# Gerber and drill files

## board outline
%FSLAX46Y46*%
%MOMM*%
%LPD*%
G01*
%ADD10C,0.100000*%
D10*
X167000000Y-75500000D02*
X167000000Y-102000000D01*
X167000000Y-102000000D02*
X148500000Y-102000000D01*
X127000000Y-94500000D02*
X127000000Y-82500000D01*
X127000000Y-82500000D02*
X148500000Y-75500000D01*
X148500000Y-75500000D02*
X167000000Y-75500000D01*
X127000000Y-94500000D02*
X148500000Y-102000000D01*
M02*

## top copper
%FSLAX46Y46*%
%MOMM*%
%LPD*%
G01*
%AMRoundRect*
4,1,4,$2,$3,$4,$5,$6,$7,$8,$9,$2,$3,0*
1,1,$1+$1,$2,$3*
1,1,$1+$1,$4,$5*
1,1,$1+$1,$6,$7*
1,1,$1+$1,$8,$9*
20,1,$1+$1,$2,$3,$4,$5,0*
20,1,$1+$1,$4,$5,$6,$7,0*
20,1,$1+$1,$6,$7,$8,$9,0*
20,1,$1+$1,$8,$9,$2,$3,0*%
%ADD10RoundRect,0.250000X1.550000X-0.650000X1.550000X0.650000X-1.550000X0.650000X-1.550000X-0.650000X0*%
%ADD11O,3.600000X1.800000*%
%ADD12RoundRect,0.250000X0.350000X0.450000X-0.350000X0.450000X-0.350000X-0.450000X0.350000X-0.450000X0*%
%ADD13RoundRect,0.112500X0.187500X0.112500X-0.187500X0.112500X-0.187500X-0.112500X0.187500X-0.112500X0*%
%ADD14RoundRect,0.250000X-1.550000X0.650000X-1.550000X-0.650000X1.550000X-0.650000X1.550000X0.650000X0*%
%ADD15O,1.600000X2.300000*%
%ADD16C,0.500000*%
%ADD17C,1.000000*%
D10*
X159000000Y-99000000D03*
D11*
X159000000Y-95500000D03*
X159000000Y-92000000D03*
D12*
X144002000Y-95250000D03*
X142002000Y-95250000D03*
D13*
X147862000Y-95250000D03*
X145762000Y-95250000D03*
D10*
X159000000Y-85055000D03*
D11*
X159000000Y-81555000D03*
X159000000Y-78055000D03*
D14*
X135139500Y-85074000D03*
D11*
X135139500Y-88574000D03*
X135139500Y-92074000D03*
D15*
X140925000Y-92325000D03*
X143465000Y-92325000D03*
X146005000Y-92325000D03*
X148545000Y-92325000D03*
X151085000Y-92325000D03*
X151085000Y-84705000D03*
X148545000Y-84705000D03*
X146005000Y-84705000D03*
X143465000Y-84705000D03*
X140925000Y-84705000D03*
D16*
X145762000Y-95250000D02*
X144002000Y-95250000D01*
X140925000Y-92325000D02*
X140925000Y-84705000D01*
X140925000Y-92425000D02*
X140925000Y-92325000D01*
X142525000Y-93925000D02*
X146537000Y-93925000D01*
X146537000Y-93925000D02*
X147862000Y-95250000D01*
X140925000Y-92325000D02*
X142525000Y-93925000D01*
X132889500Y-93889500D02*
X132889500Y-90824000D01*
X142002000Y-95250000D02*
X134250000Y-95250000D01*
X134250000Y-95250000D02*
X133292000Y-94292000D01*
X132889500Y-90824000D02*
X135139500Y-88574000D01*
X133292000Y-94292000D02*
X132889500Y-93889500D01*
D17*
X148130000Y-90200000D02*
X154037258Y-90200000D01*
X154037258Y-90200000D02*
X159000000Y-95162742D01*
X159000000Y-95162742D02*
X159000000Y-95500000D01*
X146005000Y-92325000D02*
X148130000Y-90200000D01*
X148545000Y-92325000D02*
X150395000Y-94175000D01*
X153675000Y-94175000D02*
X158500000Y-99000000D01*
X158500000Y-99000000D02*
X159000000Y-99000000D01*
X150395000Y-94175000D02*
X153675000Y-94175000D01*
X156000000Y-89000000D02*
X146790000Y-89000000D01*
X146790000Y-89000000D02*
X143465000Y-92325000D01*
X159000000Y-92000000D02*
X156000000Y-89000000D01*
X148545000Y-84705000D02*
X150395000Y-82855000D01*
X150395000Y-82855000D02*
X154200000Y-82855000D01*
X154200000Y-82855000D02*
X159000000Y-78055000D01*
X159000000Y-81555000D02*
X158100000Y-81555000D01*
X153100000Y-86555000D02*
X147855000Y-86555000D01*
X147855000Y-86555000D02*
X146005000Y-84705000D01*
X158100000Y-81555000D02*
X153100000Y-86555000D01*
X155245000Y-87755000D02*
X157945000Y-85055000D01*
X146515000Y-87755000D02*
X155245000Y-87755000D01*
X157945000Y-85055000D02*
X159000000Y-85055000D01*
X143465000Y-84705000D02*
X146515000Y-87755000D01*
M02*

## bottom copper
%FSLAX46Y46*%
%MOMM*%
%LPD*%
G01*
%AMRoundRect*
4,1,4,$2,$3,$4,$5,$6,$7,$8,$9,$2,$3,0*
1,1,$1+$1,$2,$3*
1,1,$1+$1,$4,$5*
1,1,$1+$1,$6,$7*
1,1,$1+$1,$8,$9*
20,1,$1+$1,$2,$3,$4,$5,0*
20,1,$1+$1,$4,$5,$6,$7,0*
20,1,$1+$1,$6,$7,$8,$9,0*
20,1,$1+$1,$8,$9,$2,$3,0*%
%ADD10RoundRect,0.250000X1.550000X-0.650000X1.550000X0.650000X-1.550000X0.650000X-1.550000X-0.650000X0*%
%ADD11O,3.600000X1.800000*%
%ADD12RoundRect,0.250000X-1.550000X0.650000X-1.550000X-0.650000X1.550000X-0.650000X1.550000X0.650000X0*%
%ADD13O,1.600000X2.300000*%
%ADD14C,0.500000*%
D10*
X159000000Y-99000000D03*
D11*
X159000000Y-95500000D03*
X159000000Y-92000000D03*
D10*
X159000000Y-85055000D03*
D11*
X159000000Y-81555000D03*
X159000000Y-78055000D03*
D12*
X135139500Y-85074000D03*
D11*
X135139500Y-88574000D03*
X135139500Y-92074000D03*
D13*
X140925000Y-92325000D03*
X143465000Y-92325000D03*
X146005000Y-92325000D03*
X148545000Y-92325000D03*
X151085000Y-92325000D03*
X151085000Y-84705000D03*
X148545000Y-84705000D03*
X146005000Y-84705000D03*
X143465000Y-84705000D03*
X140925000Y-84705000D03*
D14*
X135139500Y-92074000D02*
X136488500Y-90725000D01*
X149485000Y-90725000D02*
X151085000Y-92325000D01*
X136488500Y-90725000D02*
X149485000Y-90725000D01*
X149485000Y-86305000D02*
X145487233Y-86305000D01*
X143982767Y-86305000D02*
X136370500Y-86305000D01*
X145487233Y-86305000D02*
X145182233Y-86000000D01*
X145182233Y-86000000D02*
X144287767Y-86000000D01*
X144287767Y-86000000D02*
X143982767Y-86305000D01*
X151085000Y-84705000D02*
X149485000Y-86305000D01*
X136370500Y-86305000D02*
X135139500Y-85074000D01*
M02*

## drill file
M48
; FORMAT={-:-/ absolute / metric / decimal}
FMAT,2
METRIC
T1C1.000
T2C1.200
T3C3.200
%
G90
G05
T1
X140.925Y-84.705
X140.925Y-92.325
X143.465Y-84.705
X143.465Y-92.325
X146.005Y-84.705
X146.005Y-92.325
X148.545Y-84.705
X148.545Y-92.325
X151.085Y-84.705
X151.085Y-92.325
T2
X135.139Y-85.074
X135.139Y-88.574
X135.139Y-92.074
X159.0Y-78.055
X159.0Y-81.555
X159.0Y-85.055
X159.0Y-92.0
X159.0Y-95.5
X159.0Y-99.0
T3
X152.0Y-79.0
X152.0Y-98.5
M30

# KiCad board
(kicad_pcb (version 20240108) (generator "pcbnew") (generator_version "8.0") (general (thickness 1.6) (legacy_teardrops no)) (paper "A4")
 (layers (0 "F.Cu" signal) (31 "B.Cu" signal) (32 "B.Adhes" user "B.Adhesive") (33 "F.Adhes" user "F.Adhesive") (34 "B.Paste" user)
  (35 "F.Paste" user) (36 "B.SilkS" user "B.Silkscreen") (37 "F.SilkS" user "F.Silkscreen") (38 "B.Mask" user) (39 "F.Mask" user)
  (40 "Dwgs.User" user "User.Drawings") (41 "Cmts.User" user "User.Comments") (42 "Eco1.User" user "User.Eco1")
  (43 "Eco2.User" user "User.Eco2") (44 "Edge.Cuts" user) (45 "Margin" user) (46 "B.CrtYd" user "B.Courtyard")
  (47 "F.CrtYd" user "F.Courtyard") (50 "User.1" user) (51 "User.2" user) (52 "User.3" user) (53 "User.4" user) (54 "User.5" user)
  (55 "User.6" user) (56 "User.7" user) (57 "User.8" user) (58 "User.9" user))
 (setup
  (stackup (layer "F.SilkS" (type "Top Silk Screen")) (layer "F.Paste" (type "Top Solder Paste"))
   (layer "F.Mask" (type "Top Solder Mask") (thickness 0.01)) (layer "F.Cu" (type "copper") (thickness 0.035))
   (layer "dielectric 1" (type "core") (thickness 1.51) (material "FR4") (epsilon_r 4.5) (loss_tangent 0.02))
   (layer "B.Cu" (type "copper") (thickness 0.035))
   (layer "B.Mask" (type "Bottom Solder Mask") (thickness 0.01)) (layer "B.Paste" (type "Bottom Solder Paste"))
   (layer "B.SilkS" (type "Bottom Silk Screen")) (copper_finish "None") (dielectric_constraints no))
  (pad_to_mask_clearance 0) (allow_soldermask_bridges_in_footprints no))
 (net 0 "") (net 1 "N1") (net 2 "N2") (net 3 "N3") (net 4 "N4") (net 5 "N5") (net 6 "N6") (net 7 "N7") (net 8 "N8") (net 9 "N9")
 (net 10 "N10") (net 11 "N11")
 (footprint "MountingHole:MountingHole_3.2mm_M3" (layer "F.Cu") (at 152 98.5)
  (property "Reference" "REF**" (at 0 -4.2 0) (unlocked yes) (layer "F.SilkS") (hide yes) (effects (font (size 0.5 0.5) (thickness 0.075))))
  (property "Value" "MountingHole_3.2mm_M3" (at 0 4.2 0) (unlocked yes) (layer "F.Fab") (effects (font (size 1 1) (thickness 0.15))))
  (pad "" np_thru_hole circle (at 0 0) (size 3.2 3.2) (drill 3.2) (layers "*.Cu" "*.Mask")))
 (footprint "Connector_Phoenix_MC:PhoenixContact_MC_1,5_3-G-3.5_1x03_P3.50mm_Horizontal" (layer "F.Cu") (at 159 99 90)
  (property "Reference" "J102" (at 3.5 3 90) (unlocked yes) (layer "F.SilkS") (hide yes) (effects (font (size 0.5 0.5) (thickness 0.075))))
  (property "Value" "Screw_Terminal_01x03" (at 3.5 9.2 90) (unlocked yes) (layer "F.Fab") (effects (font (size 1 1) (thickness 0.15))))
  (pad "1" thru_hole roundrect (at 0 0 90) (size 1.8 3.6) (drill 1.2) (layers "*.Cu" "*.Mask") (remove_unused_layers no)
   (roundrect_rratio 0.138889) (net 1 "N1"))
  (pad "2" thru_hole oval (at 3.5 0 90) (size 1.8 3.6) (drill 1.2) (layers "*.Cu" "*.Mask") (remove_unused_layers no) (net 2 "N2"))
  (pad "3" thru_hole oval (at 7 0 90) (size 1.8 3.6) (drill 1.2) (layers "*.Cu" "*.Mask") (remove_unused_layers no) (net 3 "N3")))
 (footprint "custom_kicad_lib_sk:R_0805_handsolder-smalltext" (layer "F.Cu") (at 143.002 95.25 180)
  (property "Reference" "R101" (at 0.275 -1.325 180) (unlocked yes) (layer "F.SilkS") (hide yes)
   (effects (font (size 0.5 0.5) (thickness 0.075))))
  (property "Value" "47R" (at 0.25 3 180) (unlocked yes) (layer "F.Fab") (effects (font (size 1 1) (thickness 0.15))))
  (pad "1" smd roundrect (at -1 0 180) (size 1.2 1.4) (layers "F.Cu" "F.Paste" "F.Mask") (roundrect_rratio 0.208333) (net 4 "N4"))
  (pad "2" smd roundrect (at 1 0 180) (size 1.2 1.4) (layers "F.Cu" "F.Paste" "F.Mask") (roundrect_rratio 0.208333) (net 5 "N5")))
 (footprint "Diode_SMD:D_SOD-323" (layer "F.Cu") (at 146.812 95.25 180)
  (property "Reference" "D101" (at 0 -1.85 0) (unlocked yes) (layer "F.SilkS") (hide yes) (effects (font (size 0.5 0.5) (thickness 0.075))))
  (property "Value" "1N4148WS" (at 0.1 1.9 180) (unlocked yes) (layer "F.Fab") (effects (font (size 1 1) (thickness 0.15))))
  (pad "1" smd roundrect (at -1.05 0 180) (size 0.6 0.45) (layers "F.Cu" "F.Paste" "F.Mask") (roundrect_rratio 0.25) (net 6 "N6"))
  (pad "2" smd roundrect (at 1.05 0 180) (size 0.6 0.45) (layers "F.Cu" "F.Paste" "F.Mask") (roundrect_rratio 0.25) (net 4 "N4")))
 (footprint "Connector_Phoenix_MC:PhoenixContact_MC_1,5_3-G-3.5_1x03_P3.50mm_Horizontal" (layer "F.Cu") (at 159 85.055 90)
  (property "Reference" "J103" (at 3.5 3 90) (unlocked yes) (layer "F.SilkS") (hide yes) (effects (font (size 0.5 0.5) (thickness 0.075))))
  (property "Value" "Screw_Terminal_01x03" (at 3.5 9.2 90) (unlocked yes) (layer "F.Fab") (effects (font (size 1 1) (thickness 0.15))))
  (pad "1" thru_hole roundrect (at 0 0 90) (size 1.8 3.6) (drill 1.2) (layers "*.Cu" "*.Mask") (remove_unused_layers no)
   (roundrect_rratio 0.138889) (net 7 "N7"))
  (pad "2" thru_hole oval (at 3.5 0 90) (size 1.8 3.6) (drill 1.2) (layers "*.Cu" "*.Mask") (remove_unused_layers no) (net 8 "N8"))
  (pad "3" thru_hole oval (at 7 0 90) (size 1.8 3.6) (drill 1.2) (layers "*.Cu" "*.Mask") (remove_unused_layers no) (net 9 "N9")))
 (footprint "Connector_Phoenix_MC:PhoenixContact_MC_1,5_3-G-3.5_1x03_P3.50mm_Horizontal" (layer "F.Cu") (at 135.1395 85.074 -90)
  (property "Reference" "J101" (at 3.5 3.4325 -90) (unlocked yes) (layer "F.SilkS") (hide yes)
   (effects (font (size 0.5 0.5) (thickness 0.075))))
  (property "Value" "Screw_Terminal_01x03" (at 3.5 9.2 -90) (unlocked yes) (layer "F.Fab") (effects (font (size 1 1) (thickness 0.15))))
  (pad "1" thru_hole roundrect (at 0 0 270) (size 1.8 3.6) (drill 1.2) (layers "*.Cu" "*.Mask") (remove_unused_layers no)
   (roundrect_rratio 0.138889) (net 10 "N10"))
  (pad "2" thru_hole oval (at 3.5 0 270) (size 1.8 3.6) (drill 1.2) (layers "*.Cu" "*.Mask") (remove_unused_layers no) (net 5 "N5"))
  (pad "3" thru_hole oval (at 7 0 270) (size 1.8 3.6) (drill 1.2) (layers "*.Cu" "*.Mask") (remove_unused_layers no) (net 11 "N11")))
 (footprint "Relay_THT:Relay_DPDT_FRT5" (layer "F.Cu") (at 140.925 92.325 90)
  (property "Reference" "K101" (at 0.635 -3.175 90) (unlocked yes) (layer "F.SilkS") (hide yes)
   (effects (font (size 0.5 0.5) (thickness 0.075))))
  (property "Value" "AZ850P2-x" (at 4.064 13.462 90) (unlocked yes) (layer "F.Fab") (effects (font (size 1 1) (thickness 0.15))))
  (pad "1" thru_hole oval (at 0 0 90) (size 2.3 1.6) (drill 1) (layers "*.Cu" "*.Mask") (remove_unused_layers no) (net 6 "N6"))
  (pad "2" thru_hole oval (at 0 2.54 90) (size 2.3 1.6) (drill 1) (layers "*.Cu" "*.Mask") (remove_unused_layers no) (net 3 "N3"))
  (pad "3" thru_hole oval (at 0 5.08 90) (size 2.3 1.6) (drill 1) (layers "*.Cu" "*.Mask") (remove_unused_layers no) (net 2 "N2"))
  (pad "4" thru_hole oval (at 0 7.62 90) (size 2.3 1.6) (drill 1) (layers "*.Cu" "*.Mask") (remove_unused_layers no) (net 1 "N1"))
  (pad "5" thru_hole oval (at 0 10.16 90) (size 2.3 1.6) (drill 1) (layers "*.Cu" "*.Mask") (remove_unused_layers no) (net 11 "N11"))
  (pad "6" thru_hole oval (at 7.62 10.16 90) (size 2.3 1.6) (drill 1) (layers "*.Cu" "*.Mask") (remove_unused_layers no) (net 10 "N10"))
  (pad "7" thru_hole oval (at 7.62 7.62 90) (size 2.3 1.6) (drill 1) (layers "*.Cu" "*.Mask") (remove_unused_layers no) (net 9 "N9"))
  (pad "8" thru_hole oval (at 7.62 5.08 90) (size 2.3 1.6) (drill 1) (layers "*.Cu" "*.Mask") (remove_unused_layers no) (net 8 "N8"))
  (pad "9" thru_hole oval (at 7.62 2.54 90) (size 2.3 1.6) (drill 1) (layers "*.Cu" "*.Mask") (remove_unused_layers no) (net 7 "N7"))
  (pad "10" thru_hole oval (at 7.62 0 90) (size 2.3 1.6) (drill 1) (layers "*.Cu" "*.Mask") (remove_unused_layers no) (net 6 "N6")))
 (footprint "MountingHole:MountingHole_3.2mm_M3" (layer "F.Cu") (at 152 79)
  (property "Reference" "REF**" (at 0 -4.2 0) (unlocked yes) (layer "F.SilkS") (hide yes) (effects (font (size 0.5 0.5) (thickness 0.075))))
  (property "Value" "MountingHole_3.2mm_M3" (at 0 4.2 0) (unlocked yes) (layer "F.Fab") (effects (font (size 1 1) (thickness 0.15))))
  (pad "" np_thru_hole circle (at 0 0) (size 3.2 3.2) (drill 3.2) (layers "F&B.Cu" "*.Mask")))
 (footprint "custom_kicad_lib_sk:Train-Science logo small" (layer "B.Cu") (at 160 89 90)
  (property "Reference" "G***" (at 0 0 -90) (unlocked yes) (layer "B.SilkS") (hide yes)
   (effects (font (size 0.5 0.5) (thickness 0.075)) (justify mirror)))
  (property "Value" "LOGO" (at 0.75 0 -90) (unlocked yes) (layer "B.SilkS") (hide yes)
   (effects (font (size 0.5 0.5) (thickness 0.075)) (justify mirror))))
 (gr_line (start 167 75.5) (end 167 102) (stroke (width 0.1) (type default)) (layer "Edge.Cuts"))
 (gr_line (start 167 102) (end 148.5 102) (stroke (width 0.1) (type default)) (layer "Edge.Cuts"))
 (gr_line (start 127 94.5) (end 127 82.5) (stroke (width 0.1) (type default)) (layer "Edge.Cuts"))
 (gr_line (start 127 82.5) (end 148.5 75.5) (stroke (width 0.1) (type default)) (layer "Edge.Cuts"))
 (gr_line (start 148.5 75.5) (end 167 75.5) (stroke (width 0.1) (type default)) (layer "Edge.Cuts"))
 (gr_line (start 127 94.5) (end 148.5 102) (stroke (width 0.1) (type default)) (layer "Edge.Cuts"))
 (segment (start 145.762 95.25) (end 144.002 95.25) (width 0.5) (layer "F.Cu") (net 4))
 (segment (start 140.925 92.325) (end 140.925 84.705) (width 0.5) (layer "F.Cu") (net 6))
 (segment (start 140.925 92.425) (end 140.925 92.325) (width 0.5) (layer "F.Cu") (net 6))
 (segment (start 142.525 93.925) (end 146.537 93.925) (width 0.5) (layer "F.Cu") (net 6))
 (segment (start 146.537 93.925) (end 147.862 95.25) (width 0.5) (layer "F.Cu") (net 6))
 (segment (start 140.925 92.325) (end 142.525 93.925) (width 0.5) (layer "F.Cu") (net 6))
 (segment (start 135.1395 92.074) (end 136.4885 90.725) (width 0.5) (layer "B.Cu") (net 11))
 (segment (start 149.485 90.725) (end 151.085 92.325) (width 0.5) (layer "B.Cu") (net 11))
 (segment (start 136.4885 90.725) (end 149.485 90.725) (width 0.5) (layer "B.Cu") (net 11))
 (segment (start 149.485 86.305) (end 145.487233 86.305) (width 0.5) (layer "B.Cu") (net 10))
 (segment (start 143.982767 86.305) (end 136.3705 86.305) (width 0.5) (layer "B.Cu") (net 10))
 (segment (start 145.487233 86.305) (end 145.182233 86) (width 0.5) (layer "B.Cu") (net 10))
 (segment (start 145.182233 86) (end 144.287767 86) (width 0.5) (layer "B.Cu") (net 10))
 (segment (start 144.287767 86) (end 143.982767 86.305) (width 0.5) (layer "B.Cu") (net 10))
 (segment (start 151.085 84.705) (end 149.485 86.305) (width 0.5) (layer "B.Cu") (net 10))
 (segment (start 136.3705 86.305) (end 135.1395 85.074) (width 0.5) (layer "B.Cu") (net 10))
 (segment (start 132.8895 93.8895) (end 132.8895 90.824) (width 0.5) (layer "F.Cu") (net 5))
 (segment (start 142.002 95.25) (end 134.25 95.25) (width 0.5) (layer "F.Cu") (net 5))
 (segment (start 134.25 95.25) (end 133.292 94.292) (width 0.5) (layer "F.Cu") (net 5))
 (segment (start 132.8895 90.824) (end 135.1395 88.574) (width 0.5) (layer "F.Cu") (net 5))
 (segment (start 133.292 94.292) (end 132.8895 93.8895) (width 0.5) (layer "F.Cu") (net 5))
 (segment (start 148.13 90.2) (end 154.037258 90.2) (width 1) (layer "F.Cu") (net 2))
 (segment (start 154.037258 90.2) (end 159 95.162742) (width 1) (layer "F.Cu") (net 2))
 (segment (start 159 95.162742) (end 159 95.5) (width 1) (layer "F.Cu") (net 2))
 (segment (start 146.005 92.325) (end 148.13 90.2) (width 1) (layer "F.Cu") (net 2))
 (segment (start 148.545 92.325) (end 150.395 94.175) (width 1) (layer "F.Cu") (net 1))
 (segment (start 153.675 94.175) (end 158.5 99) (width 1) (layer "F.Cu") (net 1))
 (segment (start 158.5 99) (end 159 99) (width 1) (layer "F.Cu") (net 1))
 (segment (start 150.395 94.175) (end 153.675 94.175) (width 1) (layer "F.Cu") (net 1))
 (segment (start 156 89) (end 146.79 89) (width 1) (layer "F.Cu") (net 3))
 (segment (start 146.79 89) (end 143.465 92.325) (width 1) (layer "F.Cu") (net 3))
 (segment (start 159 92) (end 156 89) (width 1) (layer "F.Cu") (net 3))
 (segment (start 148.545 84.705) (end 150.395 82.855) (width 1) (layer "F.Cu") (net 9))
 (segment (start 150.395 82.855) (end 154.2 82.855) (width 1) (layer "F.Cu") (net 9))
 (segment (start 154.2 82.855) (end 159 78.055) (width 1) (layer "F.Cu") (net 9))
 (segment (start 159 81.555) (end 158.1 81.555) (width 1) (layer "F.Cu") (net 8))
 (segment (start 153.1 86.555) (end 147.855 86.555) (width 1) (layer "F.Cu") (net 8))
 (segment (start 147.855 86.555) (end 146.005 84.705) (width 1) (layer "F.Cu") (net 8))
 (segment (start 158.1 81.555) (end 153.1 86.555) (width 1) (layer "F.Cu") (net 8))
 (segment (start 155.245 87.755) (end 157.945 85.055) (width 1) (layer "F.Cu") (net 7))
 (segment (start 146.515 87.755) (end 155.245 87.755) (width 1) (layer "F.Cu") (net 7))
 (segment (start 157.945 85.055) (end 159 85.055) (width 1) (layer "F.Cu") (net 7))
 (segment (start 143.465 84.705) (end 146.515 87.755) (width 1) (layer "F.Cu") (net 7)))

